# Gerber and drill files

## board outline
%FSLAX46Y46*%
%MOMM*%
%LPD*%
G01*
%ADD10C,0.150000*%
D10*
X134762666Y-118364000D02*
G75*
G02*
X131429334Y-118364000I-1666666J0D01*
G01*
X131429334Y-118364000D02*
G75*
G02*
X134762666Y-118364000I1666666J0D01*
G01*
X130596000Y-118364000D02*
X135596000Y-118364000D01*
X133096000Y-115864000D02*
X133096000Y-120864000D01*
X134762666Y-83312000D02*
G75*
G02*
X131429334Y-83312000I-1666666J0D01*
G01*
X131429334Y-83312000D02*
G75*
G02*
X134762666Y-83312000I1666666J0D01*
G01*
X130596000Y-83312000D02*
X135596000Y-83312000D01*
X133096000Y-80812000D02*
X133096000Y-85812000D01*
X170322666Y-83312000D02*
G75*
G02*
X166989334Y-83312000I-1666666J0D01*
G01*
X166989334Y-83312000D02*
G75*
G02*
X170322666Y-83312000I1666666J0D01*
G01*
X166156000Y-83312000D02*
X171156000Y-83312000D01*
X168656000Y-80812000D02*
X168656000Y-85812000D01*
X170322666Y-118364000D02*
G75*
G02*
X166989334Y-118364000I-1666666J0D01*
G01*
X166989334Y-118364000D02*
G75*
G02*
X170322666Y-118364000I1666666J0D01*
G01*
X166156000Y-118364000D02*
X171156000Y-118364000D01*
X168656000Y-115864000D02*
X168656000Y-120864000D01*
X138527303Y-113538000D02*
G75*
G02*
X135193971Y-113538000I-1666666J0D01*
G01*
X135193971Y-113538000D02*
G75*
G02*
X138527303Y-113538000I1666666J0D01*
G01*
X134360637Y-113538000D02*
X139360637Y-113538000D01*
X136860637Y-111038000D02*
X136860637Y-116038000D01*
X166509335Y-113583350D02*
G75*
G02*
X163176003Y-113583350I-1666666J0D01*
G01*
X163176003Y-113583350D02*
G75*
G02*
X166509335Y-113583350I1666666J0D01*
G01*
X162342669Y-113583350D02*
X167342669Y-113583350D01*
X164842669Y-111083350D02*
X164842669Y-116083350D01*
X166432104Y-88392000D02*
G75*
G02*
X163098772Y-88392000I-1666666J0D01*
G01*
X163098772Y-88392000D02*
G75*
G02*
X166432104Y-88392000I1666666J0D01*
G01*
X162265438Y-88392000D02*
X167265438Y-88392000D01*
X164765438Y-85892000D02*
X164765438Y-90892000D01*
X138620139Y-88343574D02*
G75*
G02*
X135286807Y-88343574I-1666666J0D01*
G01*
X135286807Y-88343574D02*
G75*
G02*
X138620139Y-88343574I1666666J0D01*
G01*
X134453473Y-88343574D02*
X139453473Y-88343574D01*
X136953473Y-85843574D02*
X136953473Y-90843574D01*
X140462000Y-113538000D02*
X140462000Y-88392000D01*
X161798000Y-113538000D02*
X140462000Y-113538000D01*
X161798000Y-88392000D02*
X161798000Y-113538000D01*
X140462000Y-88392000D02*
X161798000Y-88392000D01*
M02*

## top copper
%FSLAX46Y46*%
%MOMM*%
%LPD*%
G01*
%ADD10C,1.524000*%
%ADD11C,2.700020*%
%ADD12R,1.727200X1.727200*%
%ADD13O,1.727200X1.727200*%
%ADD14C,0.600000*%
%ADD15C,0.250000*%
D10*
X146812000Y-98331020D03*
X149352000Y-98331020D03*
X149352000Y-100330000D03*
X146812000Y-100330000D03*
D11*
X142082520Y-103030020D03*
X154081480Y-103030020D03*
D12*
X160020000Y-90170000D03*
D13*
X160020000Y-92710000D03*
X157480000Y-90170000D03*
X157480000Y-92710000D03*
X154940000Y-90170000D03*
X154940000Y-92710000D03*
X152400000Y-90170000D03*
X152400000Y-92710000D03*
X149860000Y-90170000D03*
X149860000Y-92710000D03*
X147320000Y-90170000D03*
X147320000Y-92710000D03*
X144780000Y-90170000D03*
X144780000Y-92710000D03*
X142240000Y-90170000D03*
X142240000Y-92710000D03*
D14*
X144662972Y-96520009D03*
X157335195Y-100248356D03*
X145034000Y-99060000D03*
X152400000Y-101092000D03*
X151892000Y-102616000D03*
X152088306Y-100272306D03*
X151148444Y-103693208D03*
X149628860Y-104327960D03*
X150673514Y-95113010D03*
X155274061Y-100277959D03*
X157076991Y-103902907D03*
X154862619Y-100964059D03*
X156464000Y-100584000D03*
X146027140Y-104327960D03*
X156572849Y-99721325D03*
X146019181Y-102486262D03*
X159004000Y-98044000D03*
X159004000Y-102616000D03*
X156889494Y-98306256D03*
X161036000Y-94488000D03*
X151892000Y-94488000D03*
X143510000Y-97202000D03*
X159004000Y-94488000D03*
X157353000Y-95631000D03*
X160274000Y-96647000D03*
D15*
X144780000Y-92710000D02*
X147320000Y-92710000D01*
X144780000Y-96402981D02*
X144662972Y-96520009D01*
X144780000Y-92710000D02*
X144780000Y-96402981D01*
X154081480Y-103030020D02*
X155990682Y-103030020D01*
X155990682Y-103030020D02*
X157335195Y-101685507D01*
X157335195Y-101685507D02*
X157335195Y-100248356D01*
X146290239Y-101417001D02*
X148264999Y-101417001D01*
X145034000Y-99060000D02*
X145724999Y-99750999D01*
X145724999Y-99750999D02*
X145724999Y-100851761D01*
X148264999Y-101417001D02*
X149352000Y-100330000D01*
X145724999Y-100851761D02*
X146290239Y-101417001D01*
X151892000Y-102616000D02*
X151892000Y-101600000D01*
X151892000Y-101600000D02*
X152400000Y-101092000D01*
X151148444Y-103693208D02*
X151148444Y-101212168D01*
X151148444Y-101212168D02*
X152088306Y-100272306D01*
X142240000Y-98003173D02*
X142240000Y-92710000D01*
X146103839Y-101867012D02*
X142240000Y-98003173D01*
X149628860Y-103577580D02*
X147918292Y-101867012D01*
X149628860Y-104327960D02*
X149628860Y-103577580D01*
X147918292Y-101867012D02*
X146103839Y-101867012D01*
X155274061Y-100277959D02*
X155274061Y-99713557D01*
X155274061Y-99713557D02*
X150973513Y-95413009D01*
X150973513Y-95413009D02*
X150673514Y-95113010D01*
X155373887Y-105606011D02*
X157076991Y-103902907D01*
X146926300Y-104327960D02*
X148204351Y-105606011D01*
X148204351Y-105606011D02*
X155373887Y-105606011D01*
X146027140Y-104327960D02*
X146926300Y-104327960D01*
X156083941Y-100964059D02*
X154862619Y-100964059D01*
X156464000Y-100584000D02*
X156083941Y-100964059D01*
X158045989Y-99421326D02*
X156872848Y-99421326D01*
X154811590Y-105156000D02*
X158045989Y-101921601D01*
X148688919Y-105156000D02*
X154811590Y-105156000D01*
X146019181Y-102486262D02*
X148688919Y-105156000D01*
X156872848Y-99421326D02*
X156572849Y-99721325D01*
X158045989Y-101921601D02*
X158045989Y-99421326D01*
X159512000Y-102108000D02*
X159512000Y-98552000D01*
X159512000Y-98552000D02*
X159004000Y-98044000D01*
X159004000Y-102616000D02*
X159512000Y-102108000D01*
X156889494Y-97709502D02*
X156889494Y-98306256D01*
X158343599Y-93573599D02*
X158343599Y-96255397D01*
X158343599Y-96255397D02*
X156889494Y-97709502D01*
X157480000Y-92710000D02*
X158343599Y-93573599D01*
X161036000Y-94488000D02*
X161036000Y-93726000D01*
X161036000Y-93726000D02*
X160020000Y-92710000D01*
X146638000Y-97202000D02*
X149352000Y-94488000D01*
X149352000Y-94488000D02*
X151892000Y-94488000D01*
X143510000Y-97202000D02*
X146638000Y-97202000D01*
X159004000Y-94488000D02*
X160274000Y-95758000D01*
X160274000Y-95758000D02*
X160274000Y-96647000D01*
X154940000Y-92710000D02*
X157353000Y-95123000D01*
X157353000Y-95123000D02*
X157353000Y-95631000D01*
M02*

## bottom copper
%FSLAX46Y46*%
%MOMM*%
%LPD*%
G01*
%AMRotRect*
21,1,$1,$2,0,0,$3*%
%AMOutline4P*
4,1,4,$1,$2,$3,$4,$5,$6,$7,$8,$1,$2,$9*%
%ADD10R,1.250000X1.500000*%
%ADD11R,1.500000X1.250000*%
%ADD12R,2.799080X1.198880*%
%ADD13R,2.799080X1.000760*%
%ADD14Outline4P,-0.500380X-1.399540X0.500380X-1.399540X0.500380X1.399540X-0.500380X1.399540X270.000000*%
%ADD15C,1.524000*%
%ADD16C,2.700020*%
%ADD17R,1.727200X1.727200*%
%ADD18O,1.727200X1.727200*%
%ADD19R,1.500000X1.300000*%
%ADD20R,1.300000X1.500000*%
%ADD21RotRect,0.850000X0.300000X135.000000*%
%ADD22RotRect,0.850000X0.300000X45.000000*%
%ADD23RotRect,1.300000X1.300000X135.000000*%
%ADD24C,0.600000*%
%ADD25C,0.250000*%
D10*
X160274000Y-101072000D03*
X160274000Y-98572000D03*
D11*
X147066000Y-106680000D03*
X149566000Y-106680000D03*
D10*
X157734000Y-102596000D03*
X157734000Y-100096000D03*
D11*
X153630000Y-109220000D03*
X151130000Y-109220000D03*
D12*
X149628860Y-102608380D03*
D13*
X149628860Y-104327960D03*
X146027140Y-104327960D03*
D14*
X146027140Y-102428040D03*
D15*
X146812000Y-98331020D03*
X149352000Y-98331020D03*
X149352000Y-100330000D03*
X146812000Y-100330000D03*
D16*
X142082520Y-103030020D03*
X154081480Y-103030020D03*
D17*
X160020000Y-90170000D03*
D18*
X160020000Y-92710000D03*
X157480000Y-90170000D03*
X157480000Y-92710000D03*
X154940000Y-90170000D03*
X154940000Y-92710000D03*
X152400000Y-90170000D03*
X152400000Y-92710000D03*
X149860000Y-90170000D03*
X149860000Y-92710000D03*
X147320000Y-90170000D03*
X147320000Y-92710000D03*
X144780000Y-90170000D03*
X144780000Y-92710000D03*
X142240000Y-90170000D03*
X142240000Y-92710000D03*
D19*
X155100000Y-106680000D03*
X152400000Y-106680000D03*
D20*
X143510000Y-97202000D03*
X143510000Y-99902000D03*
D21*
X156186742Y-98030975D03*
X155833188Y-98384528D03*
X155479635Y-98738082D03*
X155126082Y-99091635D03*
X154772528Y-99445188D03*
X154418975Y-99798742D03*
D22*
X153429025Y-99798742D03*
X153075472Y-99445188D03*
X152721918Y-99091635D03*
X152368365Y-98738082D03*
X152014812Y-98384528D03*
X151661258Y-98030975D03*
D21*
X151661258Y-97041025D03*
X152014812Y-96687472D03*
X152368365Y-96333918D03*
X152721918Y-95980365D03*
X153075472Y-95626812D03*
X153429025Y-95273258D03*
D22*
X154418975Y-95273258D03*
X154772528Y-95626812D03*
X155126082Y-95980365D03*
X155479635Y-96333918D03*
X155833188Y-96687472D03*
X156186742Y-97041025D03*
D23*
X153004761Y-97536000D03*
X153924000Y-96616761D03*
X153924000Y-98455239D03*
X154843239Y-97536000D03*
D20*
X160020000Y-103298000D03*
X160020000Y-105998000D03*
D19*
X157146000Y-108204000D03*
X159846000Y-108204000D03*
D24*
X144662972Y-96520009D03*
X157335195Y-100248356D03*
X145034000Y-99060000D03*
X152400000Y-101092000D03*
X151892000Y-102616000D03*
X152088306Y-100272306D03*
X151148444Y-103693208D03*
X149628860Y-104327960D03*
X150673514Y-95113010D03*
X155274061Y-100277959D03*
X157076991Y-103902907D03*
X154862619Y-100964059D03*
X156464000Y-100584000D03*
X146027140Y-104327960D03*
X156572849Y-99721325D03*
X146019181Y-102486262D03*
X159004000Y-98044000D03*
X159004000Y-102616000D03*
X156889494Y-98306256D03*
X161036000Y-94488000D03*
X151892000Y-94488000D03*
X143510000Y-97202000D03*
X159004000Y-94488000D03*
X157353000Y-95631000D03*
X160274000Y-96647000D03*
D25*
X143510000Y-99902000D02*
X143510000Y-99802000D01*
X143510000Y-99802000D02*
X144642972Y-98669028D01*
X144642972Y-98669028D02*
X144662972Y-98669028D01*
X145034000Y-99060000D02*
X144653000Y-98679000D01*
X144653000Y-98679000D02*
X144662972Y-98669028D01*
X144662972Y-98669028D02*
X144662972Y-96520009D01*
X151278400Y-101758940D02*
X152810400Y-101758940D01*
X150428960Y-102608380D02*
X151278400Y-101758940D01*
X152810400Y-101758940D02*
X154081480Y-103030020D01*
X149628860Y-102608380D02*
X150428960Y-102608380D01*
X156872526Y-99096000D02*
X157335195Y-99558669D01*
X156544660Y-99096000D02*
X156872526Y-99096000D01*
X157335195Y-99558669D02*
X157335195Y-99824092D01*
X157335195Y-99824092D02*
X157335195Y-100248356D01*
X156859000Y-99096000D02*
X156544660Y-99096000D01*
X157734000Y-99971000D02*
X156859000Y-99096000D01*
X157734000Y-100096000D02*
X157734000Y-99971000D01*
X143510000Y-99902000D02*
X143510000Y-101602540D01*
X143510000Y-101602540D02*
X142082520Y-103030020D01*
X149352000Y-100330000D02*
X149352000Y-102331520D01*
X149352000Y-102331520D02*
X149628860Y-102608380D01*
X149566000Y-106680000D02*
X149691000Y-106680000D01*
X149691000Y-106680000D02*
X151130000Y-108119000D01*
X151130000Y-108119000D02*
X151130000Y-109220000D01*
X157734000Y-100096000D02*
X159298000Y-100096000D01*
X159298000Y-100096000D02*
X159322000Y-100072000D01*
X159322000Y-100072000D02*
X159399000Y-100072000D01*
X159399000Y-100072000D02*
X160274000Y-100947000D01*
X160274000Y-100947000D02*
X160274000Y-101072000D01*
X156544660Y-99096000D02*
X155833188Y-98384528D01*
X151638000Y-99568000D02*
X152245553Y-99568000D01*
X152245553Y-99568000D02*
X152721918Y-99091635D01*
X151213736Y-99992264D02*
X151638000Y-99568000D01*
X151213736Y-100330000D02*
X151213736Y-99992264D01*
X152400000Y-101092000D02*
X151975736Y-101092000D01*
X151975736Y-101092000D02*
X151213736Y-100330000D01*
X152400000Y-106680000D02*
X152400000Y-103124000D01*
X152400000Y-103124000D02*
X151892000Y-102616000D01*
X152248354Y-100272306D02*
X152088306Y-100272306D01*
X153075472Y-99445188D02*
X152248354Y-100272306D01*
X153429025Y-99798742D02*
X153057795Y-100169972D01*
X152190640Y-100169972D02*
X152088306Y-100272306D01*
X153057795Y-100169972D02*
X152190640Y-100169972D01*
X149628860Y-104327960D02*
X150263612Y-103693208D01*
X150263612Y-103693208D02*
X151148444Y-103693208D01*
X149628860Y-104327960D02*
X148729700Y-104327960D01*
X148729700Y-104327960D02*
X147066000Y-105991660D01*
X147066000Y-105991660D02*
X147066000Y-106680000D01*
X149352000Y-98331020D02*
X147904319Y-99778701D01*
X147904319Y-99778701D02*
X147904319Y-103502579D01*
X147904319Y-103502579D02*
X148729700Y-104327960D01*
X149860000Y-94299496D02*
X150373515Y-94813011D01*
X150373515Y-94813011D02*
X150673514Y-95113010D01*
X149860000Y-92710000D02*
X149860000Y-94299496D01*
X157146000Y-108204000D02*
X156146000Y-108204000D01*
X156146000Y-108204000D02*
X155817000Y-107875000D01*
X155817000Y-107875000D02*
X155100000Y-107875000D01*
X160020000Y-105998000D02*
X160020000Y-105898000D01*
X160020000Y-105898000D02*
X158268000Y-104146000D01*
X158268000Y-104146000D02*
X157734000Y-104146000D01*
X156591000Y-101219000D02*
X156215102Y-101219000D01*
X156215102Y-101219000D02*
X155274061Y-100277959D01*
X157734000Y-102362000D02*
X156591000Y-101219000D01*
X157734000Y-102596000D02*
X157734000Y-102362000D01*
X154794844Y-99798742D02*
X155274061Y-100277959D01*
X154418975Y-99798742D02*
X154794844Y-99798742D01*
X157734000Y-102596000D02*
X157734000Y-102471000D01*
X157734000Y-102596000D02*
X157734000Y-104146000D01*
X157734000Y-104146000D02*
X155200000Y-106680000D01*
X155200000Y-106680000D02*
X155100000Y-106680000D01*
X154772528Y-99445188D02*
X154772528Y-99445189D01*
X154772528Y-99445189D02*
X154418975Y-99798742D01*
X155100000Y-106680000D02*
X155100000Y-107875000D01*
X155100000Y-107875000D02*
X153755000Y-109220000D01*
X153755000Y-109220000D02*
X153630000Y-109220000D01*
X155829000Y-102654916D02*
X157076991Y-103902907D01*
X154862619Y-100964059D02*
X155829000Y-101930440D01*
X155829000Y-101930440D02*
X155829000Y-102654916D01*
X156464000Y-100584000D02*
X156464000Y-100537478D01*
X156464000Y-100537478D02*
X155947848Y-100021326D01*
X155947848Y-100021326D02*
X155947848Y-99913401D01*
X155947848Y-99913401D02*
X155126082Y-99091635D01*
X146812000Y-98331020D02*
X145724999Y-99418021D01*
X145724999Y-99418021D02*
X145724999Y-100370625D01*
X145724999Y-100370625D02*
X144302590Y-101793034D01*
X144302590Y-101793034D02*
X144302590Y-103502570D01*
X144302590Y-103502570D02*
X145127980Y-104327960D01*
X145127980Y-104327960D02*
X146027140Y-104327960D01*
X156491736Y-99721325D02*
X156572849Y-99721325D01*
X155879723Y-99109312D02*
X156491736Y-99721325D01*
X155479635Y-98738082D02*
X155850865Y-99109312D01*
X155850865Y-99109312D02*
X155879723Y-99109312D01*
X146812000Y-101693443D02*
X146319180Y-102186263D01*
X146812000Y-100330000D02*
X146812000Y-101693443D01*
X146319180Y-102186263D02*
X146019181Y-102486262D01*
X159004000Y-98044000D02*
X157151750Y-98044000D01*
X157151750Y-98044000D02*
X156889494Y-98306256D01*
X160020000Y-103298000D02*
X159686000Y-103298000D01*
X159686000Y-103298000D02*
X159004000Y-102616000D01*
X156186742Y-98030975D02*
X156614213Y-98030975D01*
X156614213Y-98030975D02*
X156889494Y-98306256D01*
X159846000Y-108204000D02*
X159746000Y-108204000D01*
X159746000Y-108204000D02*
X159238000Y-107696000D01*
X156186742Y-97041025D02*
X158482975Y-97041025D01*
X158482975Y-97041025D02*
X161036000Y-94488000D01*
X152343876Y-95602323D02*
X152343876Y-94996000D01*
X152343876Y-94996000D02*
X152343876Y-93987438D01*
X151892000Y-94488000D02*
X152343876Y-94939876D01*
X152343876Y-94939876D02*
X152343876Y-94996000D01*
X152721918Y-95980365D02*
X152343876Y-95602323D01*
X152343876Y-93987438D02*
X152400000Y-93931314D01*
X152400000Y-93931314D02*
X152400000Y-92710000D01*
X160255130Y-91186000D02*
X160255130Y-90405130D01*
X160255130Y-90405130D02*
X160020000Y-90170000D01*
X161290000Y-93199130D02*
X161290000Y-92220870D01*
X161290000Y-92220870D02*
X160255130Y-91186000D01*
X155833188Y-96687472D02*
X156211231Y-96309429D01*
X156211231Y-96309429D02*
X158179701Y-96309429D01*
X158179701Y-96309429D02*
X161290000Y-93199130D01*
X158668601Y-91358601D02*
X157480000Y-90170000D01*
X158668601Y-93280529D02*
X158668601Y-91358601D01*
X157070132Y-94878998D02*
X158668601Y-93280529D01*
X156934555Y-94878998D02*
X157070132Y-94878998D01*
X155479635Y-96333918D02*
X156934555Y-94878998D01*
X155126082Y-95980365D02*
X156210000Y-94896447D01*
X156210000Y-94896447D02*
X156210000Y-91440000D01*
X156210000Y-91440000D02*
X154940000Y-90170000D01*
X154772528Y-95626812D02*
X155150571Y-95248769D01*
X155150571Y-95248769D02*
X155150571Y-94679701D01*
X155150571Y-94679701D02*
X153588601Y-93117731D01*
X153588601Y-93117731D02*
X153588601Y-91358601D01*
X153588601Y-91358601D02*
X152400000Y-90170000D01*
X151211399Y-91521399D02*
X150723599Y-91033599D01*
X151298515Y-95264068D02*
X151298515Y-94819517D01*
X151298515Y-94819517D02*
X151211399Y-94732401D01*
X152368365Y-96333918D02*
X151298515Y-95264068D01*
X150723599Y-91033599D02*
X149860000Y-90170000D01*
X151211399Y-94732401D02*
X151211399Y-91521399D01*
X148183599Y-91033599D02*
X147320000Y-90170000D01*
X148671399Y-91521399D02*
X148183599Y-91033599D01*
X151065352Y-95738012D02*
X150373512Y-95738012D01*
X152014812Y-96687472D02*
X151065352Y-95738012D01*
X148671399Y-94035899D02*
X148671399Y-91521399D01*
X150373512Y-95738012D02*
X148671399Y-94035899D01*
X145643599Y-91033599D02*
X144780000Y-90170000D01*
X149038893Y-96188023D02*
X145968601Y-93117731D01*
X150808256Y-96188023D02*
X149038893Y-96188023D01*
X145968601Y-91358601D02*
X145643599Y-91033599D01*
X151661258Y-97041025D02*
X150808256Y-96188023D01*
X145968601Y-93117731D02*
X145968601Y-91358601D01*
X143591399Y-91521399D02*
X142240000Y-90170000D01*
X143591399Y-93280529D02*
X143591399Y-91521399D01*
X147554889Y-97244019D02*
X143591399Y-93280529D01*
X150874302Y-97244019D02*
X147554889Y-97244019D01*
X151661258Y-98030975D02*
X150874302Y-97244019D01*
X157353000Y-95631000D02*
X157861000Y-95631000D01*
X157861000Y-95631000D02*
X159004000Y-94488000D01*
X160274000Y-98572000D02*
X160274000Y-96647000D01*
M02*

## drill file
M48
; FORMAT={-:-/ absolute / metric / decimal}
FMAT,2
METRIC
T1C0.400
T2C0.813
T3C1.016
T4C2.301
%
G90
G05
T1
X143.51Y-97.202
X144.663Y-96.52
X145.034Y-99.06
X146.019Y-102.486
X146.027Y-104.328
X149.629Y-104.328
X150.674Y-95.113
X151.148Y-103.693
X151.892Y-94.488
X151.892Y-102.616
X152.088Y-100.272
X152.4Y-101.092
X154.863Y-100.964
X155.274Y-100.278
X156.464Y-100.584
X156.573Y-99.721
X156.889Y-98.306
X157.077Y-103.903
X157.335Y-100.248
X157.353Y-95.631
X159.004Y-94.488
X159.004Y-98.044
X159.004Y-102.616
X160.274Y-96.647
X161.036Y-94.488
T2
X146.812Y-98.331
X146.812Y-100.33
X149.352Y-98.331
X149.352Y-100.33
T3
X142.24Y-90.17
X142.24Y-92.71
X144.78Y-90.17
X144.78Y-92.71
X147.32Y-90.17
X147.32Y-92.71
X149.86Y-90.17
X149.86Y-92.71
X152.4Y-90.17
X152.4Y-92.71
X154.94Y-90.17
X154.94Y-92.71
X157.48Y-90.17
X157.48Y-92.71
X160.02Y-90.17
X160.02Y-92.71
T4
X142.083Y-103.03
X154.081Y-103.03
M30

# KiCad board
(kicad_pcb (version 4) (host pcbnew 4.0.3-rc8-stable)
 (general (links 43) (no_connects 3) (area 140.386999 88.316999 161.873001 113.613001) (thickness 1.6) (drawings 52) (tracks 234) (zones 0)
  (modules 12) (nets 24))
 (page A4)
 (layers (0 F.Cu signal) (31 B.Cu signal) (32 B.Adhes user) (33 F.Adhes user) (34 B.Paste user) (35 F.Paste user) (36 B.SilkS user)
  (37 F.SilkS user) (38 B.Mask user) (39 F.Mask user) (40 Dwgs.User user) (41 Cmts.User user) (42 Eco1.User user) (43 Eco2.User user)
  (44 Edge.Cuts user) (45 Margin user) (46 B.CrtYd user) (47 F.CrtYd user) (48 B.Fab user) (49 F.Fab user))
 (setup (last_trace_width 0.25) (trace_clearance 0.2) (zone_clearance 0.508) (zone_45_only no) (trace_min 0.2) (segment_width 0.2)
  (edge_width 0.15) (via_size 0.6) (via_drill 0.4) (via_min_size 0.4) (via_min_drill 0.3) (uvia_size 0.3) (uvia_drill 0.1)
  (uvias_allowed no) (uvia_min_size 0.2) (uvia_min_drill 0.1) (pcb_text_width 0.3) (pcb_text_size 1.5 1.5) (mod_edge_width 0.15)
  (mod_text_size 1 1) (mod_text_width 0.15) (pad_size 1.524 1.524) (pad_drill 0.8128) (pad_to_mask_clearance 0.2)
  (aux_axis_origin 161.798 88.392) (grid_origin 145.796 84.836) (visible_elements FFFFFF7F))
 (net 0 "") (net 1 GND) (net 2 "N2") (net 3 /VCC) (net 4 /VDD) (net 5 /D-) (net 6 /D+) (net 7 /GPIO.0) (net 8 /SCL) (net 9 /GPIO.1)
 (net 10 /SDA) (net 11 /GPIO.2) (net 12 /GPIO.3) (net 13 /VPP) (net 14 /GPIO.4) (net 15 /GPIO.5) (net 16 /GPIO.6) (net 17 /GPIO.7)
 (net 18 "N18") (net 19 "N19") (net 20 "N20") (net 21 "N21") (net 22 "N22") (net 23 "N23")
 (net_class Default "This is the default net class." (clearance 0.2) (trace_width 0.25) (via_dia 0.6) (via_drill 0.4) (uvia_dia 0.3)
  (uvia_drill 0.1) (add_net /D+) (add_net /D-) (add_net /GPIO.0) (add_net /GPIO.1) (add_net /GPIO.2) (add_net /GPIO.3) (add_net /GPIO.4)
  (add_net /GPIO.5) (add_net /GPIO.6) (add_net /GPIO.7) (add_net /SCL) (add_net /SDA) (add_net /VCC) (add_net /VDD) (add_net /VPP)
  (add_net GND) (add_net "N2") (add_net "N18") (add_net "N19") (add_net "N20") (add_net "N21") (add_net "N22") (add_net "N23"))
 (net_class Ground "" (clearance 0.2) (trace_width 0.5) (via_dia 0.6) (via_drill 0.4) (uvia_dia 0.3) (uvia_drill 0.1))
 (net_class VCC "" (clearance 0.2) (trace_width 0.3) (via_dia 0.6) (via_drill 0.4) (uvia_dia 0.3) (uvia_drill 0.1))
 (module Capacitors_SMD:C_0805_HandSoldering (layer B.Cu) (at 160.274 99.822 90)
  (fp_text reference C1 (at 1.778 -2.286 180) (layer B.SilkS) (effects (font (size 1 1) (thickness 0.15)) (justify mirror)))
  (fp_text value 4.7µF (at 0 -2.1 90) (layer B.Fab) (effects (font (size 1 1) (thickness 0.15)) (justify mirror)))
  (pad 1 smd rect (at -1.25 0 90) (size 1.5 1.25) (layers B.Cu B.Paste B.Mask) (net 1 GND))
  (pad 2 smd rect (at 1.25 0 90) (size 1.5 1.25) (layers B.Cu B.Paste B.Mask) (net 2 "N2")))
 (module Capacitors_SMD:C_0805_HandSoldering (layer B.Cu) (at 148.316 106.68)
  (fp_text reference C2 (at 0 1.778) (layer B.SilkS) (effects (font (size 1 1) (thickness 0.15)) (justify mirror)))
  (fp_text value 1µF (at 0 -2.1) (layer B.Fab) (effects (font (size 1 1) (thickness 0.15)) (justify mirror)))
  (pad 1 smd rect (at -1.25 0) (size 1.5 1.25) (layers B.Cu B.Paste B.Mask) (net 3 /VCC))
  (pad 2 smd rect (at 1.25 0) (size 1.5 1.25) (layers B.Cu B.Paste B.Mask) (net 1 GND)))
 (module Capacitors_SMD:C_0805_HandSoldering (layer B.Cu) (at 157.734 101.346 90)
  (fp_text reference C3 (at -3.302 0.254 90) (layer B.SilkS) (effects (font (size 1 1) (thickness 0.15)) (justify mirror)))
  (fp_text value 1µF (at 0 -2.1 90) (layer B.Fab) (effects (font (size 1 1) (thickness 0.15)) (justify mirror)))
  (pad 1 smd rect (at -1.25 0 90) (size 1.5 1.25) (layers B.Cu B.Paste B.Mask) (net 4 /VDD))
  (pad 2 smd rect (at 1.25 0 90) (size 1.5 1.25) (layers B.Cu B.Paste B.Mask) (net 1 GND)))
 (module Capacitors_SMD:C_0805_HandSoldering (layer B.Cu) (at 152.38 109.22 180)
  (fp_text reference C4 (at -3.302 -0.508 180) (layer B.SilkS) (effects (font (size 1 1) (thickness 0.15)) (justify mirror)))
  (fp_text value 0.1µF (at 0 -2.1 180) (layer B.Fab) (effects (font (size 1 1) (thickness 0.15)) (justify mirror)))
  (pad 1 smd rect (at -1.25 0 180) (size 1.5 1.25) (layers B.Cu B.Paste B.Mask) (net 4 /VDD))
  (pad 2 smd rect (at 1.25 0 180) (size 1.5 1.25) (layers B.Cu B.Paste B.Mask) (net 1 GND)))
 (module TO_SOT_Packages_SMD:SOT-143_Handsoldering (layer B.Cu) (at 147.828 103.378 270)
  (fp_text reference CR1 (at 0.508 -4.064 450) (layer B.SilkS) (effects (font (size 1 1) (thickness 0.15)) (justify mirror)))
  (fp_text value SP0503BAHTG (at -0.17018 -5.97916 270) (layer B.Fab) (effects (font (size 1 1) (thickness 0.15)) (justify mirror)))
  (pad 1 smd rect (at -0.76962 -1.80086 270) (size 1.19888 2.79908) (layers B.Cu B.Paste B.Mask) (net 1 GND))
  (pad 2 smd rect (at 0.94996 -1.80086 270) (size 1.00076 2.79908) (layers B.Cu B.Paste B.Mask) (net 3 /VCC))
  (pad 3 smd rect (at 0.94996 1.80086 270) (size 1.00076 2.79908) (layers B.Cu B.Paste B.Mask) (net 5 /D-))
  (pad 4 smd trapezoid (at -0.94996 1.80086 270) (size 1.00076 2.79908) (layers B.Cu B.Paste B.Mask) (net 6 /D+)))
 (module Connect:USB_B (layer F.Cu) (at 149.352 98.33102 270)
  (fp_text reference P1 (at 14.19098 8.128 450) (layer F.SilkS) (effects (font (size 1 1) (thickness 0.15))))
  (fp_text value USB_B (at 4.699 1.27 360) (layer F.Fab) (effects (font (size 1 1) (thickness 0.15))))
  (pad 2 thru_hole circle (at 0 2.54 180) (size 1.524 1.524) (drill 0.8128) (layers *.Cu *.Mask F.SilkS) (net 5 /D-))
  (pad 1 thru_hole circle (at 0 0 180) (size 1.524 1.524) (drill 0.8128) (layers *.Cu *.Mask F.SilkS) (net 3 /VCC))
  (pad 4 thru_hole circle (at 1.99898 0 180) (size 1.524 1.524) (drill 0.8128) (layers *.Cu *.Mask F.SilkS) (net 1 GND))
  (pad 3 thru_hole circle (at 1.99898 2.54 180) (size 1.524 1.524) (drill 0.8128) (layers *.Cu *.Mask F.SilkS) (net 6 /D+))
  (pad 5 thru_hole circle (at 4.699 7.26948 180) (size 2.70002 2.70002) (drill 2.30124) (layers *.Cu *.Mask F.SilkS) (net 1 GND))
  (pad 5 thru_hole circle (at 4.699 -4.72948 180) (size 2.70002 2.70002) (drill 2.30124) (layers *.Cu *.Mask F.SilkS) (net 1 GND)))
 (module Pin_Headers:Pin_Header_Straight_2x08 (layer F.Cu) (at 160.02 90.17 270)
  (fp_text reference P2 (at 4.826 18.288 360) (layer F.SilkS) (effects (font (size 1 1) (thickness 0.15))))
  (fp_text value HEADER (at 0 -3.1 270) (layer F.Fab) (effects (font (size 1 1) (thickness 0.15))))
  (pad 1 thru_hole rect (at 0 0 270) (size 1.7272 1.7272) (drill 1.016) (layers *.Cu *.Mask F.SilkS) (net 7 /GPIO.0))
  (pad 2 thru_hole oval (at 2.54 0 270) (size 1.7272 1.7272) (drill 1.016) (layers *.Cu *.Mask F.SilkS) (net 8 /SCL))
  (pad 3 thru_hole oval (at 0 2.54 270) (size 1.7272 1.7272) (drill 1.016) (layers *.Cu *.Mask F.SilkS) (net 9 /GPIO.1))
  (pad 4 thru_hole oval (at 2.54 2.54 270) (size 1.7272 1.7272) (drill 1.016) (layers *.Cu *.Mask F.SilkS) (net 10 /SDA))
  (pad 5 thru_hole oval (at 0 5.08 270) (size 1.7272 1.7272) (drill 1.016) (layers *.Cu *.Mask F.SilkS) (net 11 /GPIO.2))
  (pad 6 thru_hole oval (at 2.54 5.08 270) (size 1.7272 1.7272) (drill 1.016) (layers *.Cu *.Mask F.SilkS) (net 2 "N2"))
  (pad 7 thru_hole oval (at 0 7.62 270) (size 1.7272 1.7272) (drill 1.016) (layers *.Cu *.Mask F.SilkS) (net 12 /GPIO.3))
  (pad 8 thru_hole oval (at 2.54 7.62 270) (size 1.7272 1.7272) (drill 1.016) (layers *.Cu *.Mask F.SilkS) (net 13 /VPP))
  (pad 9 thru_hole oval (at 0 10.16 270) (size 1.7272 1.7272) (drill 1.016) (layers *.Cu *.Mask F.SilkS) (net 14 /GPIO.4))
  (pad 10 thru_hole oval (at 2.54 10.16 270) (size 1.7272 1.7272) (drill 1.016) (layers *.Cu *.Mask F.SilkS) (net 4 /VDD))
  (pad 11 thru_hole oval (at 0 12.7 270) (size 1.7272 1.7272) (drill 1.016) (layers *.Cu *.Mask F.SilkS) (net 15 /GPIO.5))
  (pad 12 thru_hole oval (at 2.54 12.7 270) (size 1.7272 1.7272) (drill 1.016) (layers *.Cu *.Mask F.SilkS) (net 1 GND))
  (pad 13 thru_hole oval (at 0 15.24 270) (size 1.7272 1.7272) (drill 1.016) (layers *.Cu *.Mask F.SilkS) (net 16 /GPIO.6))
  (pad 14 thru_hole oval (at 2.54 15.24 270) (size 1.7272 1.7272) (drill 1.016) (layers *.Cu *.Mask F.SilkS) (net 1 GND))
  (pad 15 thru_hole oval (at 0 17.78 270) (size 1.7272 1.7272) (drill 1.016) (layers *.Cu *.Mask F.SilkS) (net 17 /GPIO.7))
  (pad 16 thru_hole oval (at 2.54 17.78 270) (size 1.7272 1.7272) (drill 1.016) (layers *.Cu *.Mask F.SilkS) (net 3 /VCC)))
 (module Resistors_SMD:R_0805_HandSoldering (layer B.Cu) (at 153.75 106.68 180)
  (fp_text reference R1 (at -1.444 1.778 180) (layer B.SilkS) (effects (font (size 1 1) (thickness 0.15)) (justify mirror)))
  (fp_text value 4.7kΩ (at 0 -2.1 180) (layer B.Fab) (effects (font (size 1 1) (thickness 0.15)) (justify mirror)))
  (pad 1 smd rect (at -1.35 0 180) (size 1.5 1.3) (layers B.Cu B.Paste B.Mask) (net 4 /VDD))
  (pad 2 smd rect (at 1.35 0 180) (size 1.5 1.3) (layers B.Cu B.Paste B.Mask) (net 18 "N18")))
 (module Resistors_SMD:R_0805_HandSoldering (layer B.Cu) (at 143.51 98.552 270)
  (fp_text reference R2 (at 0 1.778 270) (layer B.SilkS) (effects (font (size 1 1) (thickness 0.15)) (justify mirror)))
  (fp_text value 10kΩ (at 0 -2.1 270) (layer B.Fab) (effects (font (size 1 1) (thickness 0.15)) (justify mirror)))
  (pad 1 smd rect (at -1.35 0 270) (size 1.5 1.3) (layers B.Cu B.Paste B.Mask) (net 13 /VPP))
  (pad 2 smd rect (at 1.35 0 270) (size 1.5 1.3) (layers B.Cu B.Paste B.Mask) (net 1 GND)))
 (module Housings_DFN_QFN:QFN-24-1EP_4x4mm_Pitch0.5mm (layer B.Cu) (at 153.924 97.536 135)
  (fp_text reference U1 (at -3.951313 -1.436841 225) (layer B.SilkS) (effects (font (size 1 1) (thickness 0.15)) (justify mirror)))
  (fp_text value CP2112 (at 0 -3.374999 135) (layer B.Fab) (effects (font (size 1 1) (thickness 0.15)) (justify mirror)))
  (pad 1 smd rect (at -1.95 1.25 135) (size 0.85 0.3) (layers B.Cu B.Paste B.Mask) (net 10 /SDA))
  (pad 2 smd rect (at -1.95 0.75 135) (size 0.85 0.3) (layers B.Cu B.Paste B.Mask) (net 1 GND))
  (pad 3 smd rect (at -1.95 0.25 135) (size 0.85 0.3) (layers B.Cu B.Paste B.Mask) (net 6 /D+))
  (pad 4 smd rect (at -1.95 -0.25 135) (size 0.85 0.3) (layers B.Cu B.Paste B.Mask) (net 5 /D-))
  (pad 5 smd rect (at -1.95 -0.75 135) (size 0.85 0.3) (layers B.Cu B.Paste B.Mask) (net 4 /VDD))
  (pad 6 smd rect (at -1.95 -1.25 135) (size 0.85 0.3) (layers B.Cu B.Paste B.Mask) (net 4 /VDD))
  (pad 7 smd rect (at -1.25 -1.95 45) (size 0.85 0.3) (layers B.Cu B.Paste B.Mask) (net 3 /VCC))
  (pad 8 smd rect (at -0.75 -1.95 45) (size 0.85 0.3) (layers B.Cu B.Paste B.Mask) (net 3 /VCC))
  (pad 9 smd rect (at -0.25 -1.95 45) (size 0.85 0.3) (layers B.Cu B.Paste B.Mask) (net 18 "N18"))
  (pad 10 smd rect (at 0.25 -1.95 45) (size 0.85 0.3) (layers B.Cu B.Paste B.Mask) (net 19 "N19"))
  (pad 11 smd rect (at 0.75 -1.95 45) (size 0.85 0.3) (layers B.Cu B.Paste B.Mask) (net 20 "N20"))
  (pad 12 smd rect (at 1.25 -1.95 45) (size 0.85 0.3) (layers B.Cu B.Paste B.Mask) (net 17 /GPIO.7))
  (pad 13 smd rect (at 1.95 -1.25 135) (size 0.85 0.3) (layers B.Cu B.Paste B.Mask) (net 16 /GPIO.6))
  (pad 14 smd rect (at 1.95 -0.75 135) (size 0.85 0.3) (layers B.Cu B.Paste B.Mask) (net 15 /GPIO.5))
  (pad 15 smd rect (at 1.95 -0.25 135) (size 0.85 0.3) (layers B.Cu B.Paste B.Mask) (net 14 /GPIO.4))
  (pad 16 smd rect (at 1.95 0.25 135) (size 0.85 0.3) (layers B.Cu B.Paste B.Mask) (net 13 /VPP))
  (pad 17 smd rect (at 1.95 0.75 135) (size 0.85 0.3) (layers B.Cu B.Paste B.Mask) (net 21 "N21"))
  (pad 18 smd rect (at 1.95 1.25 135) (size 0.85 0.3) (layers B.Cu B.Paste B.Mask) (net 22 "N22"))
  (pad 19 smd rect (at 1.25 1.95 45) (size 0.85 0.3) (layers B.Cu B.Paste B.Mask) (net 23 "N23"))
  (pad 20 smd rect (at 0.75 1.95 45) (size 0.85 0.3) (layers B.Cu B.Paste B.Mask) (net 12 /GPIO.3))
  (pad 21 smd rect (at 0.25 1.95 45) (size 0.85 0.3) (layers B.Cu B.Paste B.Mask) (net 11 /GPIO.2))
  (pad 22 smd rect (at -0.25 1.95 45) (size 0.85 0.3) (layers B.Cu B.Paste B.Mask) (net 9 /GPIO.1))
  (pad 23 smd rect (at -0.75 1.95 45) (size 0.85 0.3) (layers B.Cu B.Paste B.Mask) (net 7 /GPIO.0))
  (pad 24 smd rect (at -1.25 1.95 45) (size 0.85 0.3) (layers B.Cu B.Paste B.Mask) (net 8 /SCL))
  (pad 25 smd rect (at 0.65 -0.65 135) (size 1.3 1.3) (layers B.Cu B.Paste B.Mask) (solder_paste_margin_ratio -0.2))
  (pad 25 smd rect (at 0.65 0.65 135) (size 1.3 1.3) (layers B.Cu B.Paste B.Mask) (solder_paste_margin_ratio -0.2))
  (pad 25 smd rect (at -0.65 -0.65 135) (size 1.3 1.3) (layers B.Cu B.Paste B.Mask) (solder_paste_margin_ratio -0.2))
  (pad 25 smd rect (at -0.65 0.65 135) (size 1.3 1.3) (layers B.Cu B.Paste B.Mask) (solder_paste_margin_ratio -0.2)))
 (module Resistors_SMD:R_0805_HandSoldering (layer B.Cu) (at 160.02 104.648 270)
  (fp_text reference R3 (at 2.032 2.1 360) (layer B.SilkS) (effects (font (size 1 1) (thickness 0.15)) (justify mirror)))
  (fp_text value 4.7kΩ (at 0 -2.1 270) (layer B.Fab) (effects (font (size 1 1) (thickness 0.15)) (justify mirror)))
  (pad 1 smd rect (at -1.35 0 270) (size 1.5 1.3) (layers B.Cu B.Paste B.Mask) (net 10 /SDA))
  (pad 2 smd rect (at 1.35 0 270) (size 1.5 1.3) (layers B.Cu B.Paste B.Mask) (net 4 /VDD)))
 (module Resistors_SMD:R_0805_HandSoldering (layer B.Cu) (at 158.496 108.204)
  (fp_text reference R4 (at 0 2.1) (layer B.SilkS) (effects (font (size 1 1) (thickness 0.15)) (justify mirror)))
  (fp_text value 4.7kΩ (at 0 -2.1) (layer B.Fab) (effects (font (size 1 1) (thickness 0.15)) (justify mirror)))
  (pad 1 smd rect (at -1.35 0) (size 1.5 1.3) (layers B.Cu B.Paste B.Mask) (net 4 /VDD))
  (pad 2 smd rect (at 1.35 0) (size 1.5 1.3) (layers B.Cu B.Paste B.Mask) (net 8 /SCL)))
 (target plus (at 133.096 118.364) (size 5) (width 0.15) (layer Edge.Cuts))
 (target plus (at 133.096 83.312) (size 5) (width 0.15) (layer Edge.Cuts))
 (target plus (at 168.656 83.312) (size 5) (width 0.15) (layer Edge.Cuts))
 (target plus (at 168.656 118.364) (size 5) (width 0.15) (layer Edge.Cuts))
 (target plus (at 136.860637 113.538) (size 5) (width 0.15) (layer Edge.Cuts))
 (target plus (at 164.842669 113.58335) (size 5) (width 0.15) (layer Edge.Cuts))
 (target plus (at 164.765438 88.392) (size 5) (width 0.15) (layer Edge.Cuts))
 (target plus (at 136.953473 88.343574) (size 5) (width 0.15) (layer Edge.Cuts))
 (gr_line (start 140.462 113.538) (end 140.462 88.392) (layer Edge.Cuts) (width 0.15))
 (gr_line (start 161.798 113.538) (end 140.462 113.538) (layer Edge.Cuts) (width 0.15))
 (gr_line (start 161.798 88.392) (end 161.798 113.538) (layer Edge.Cuts) (width 0.15))
 (gr_line (start 140.462 88.392) (end 161.798 88.392) (layer Edge.Cuts) (width 0.15))
 (segment (start 143.51 99.902) (end 143.51 99.802) (width 0.25) (layer B.Cu) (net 1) (status 30))
 (segment (start 143.51 99.802) (end 144.642972 98.669028) (width 0.25) (layer B.Cu) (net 1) (status 10))
 (segment (start 144.642972 98.669028) (end 144.662972 98.669028) (width 0.25) (layer B.Cu) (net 1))
 (segment (start 145.034 99.06) (end 144.653 98.679) (width 0.25) (layer B.Cu) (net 1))
 (segment (start 144.653 98.679) (end 144.662972 98.669028) (width 0.25) (layer B.Cu) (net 1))
 (segment (start 144.662972 98.669028) (end 144.662972 96.520009) (width 0.25) (layer B.Cu) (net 1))
 (segment (start 144.78 92.71) (end 147.32 92.71) (width 0.25) (layer F.Cu) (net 1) (status 30))
 (segment (start 144.78 96.402981) (end 144.662972 96.520009) (width 0.25) (layer F.Cu) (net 1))
 (segment (start 144.78 92.71) (end 144.78 96.402981) (width 0.25) (layer F.Cu) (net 1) (status 10))
 (via (at 144.662972 96.520009) (size 0.6) (drill 0.4) (layers F.Cu B.Cu) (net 1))
 (segment (start 151.2784 101.75894) (end 152.8104 101.75894) (width 0.25) (layer B.Cu) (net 1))
 (segment (start 150.42896 102.60838) (end 151.2784 101.75894) (width 0.25) (layer B.Cu) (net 1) (status 10))
 (segment (start 152.8104 101.75894) (end 154.08148 103.03002) (width 0.25) (layer B.Cu) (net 1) (status 20))
 (segment (start 149.62886 102.60838) (end 150.42896 102.60838) (width 0.25) (layer B.Cu) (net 1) (status 30))
 (segment (start 156.872526 99.096) (end 157.335195 99.558669) (width 0.25) (layer B.Cu) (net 1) (status 20))
 (segment (start 156.54466 99.096) (end 156.872526 99.096) (width 0.25) (layer B.Cu) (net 1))
 (segment (start 157.335195 99.558669) (end 157.335195 99.824092) (width 0.25) (layer B.Cu) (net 1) (status 30))
 (segment (start 157.335195 99.824092) (end 157.335195 100.248356) (width 0.25) (layer B.Cu) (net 1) (status 30))
 (segment (start 154.08148 103.03002) (end 155.990682 103.03002) (width 0.25) (layer F.Cu) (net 1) (status 10))
 (via (at 157.335195 100.248356) (size 0.6) (drill 0.4) (layers F.Cu B.Cu) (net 1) (status 30))
 (segment (start 155.990682 103.03002) (end 157.335195 101.685507) (width 0.25) (layer F.Cu) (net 1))
 (segment (start 157.335195 101.685507) (end 157.335195 100.248356) (width 0.25) (layer F.Cu) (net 1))
 (segment (start 156.859 99.096) (end 156.54466 99.096) (width 0.25) (layer B.Cu) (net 1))
 (segment (start 157.734 99.971) (end 156.859 99.096) (width 0.25) (layer B.Cu) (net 1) (status 10))
 (segment (start 157.734 100.096) (end 157.734 99.971) (width 0.25) (layer B.Cu) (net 1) (status 30))
 (segment (start 146.290239 101.417001) (end 148.264999 101.417001) (width 0.25) (layer F.Cu) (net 1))
 (segment (start 145.034 99.06) (end 145.724999 99.750999) (width 0.25) (layer F.Cu) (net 1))
 (segment (start 145.724999 99.750999) (end 145.724999 100.851761) (width 0.25) (layer F.Cu) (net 1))
 (segment (start 148.264999 101.417001) (end 149.352 100.33) (width 0.25) (layer F.Cu) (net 1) (status 20))
 (segment (start 145.724999 100.851761) (end 146.290239 101.417001) (width 0.25) (layer F.Cu) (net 1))
 (via (at 145.034 99.06) (size 0.6) (drill 0.4) (layers F.Cu B.Cu) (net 1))
 (segment (start 143.51 99.902) (end 143.51 101.60254) (width 0.25) (layer B.Cu) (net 1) (status 10))
 (segment (start 143.51 101.60254) (end 142.08252 103.03002) (width 0.25) (layer B.Cu) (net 1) (status 20))
 (segment (start 149.352 100.33) (end 149.352 102.33152) (width 0.25) (layer B.Cu) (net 1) (status 30))
 (segment (start 149.352 102.33152) (end 149.62886 102.60838) (width 0.25) (layer B.Cu) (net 1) (status 30))
 (segment (start 149.566 106.68) (end 149.691 106.68) (width 0.25) (layer B.Cu) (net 1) (status 30))
 (segment (start 149.691 106.68) (end 151.13 108.119) (width 0.25) (layer B.Cu) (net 1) (status 10))
 (segment (start 151.13 108.119) (end 151.13 109.22) (width 0.25) (layer B.Cu) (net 1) (status 20))
 (segment (start 157.734 100.096) (end 159.298 100.096) (width 0.25) (layer B.Cu) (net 1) (status 10))
 (segment (start 159.298 100.096) (end 159.322 100.072) (width 0.25) (layer B.Cu) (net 1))
 (segment (start 159.322 100.072) (end 159.399 100.072) (width 0.25) (layer B.Cu) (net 1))
 (segment (start 159.399 100.072) (end 160.274 100.947) (width 0.25) (layer B.Cu) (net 1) (status 20))
 (segment (start 160.274 100.947) (end 160.274 101.072) (width 0.25) (layer B.Cu) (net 1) (status 30))
 (segment (start 156.54466 99.096) (end 155.833188 98.384528) (width 0.25) (layer B.Cu) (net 1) (status 20))
 (segment (start 151.638 99.568) (end 152.245553 99.568) (width 0.25) (layer B.Cu) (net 18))
 (segment (start 152.245553 99.568) (end 152.721918 99.091635) (width 0.25) (layer B.Cu) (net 18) (status 20))
 (segment (start 151.213736 99.992264) (end 151.638 99.568) (width 0.25) (layer B.Cu) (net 18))
 (segment (start 151.213736 100.33) (end 151.213736 99.992264) (width 0.25) (layer B.Cu) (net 18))
 (segment (start 152.4 101.092) (end 151.975736 101.092) (width 0.25) (layer B.Cu) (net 18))
 (segment (start 151.975736 101.092) (end 151.213736 100.33) (width 0.25) (layer B.Cu) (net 18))
 (segment (start 151.892 102.616) (end 151.892 101.6) (width 0.25) (layer F.Cu) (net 18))
 (via (at 152.4 101.092) (size 0.6) (drill 0.4) (layers F.Cu B.Cu) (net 18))
 (segment (start 151.892 101.6) (end 152.4 101.092) (width 0.25) (layer F.Cu) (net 18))
 (via (at 151.892 102.616) (size 0.6) (drill 0.4) (layers F.Cu B.Cu) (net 18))
 (segment (start 152.4 106.68) (end 152.4 103.124) (width 0.25) (layer B.Cu) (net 18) (status 10))
 (segment (start 152.4 103.124) (end 151.892 102.616) (width 0.25) (layer B.Cu) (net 18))
 (segment (start 152.248354 100.272306) (end 152.088306 100.272306) (width 0.25) (layer B.Cu) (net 3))
 (via (at 152.088306 100.272306) (size 0.6) (drill 0.4) (layers F.Cu B.Cu) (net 3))
 (segment (start 153.075472 99.445188) (end 152.248354 100.272306) (width 0.25) (layer B.Cu) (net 3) (status 10))
 (segment (start 151.148444 103.693208) (end 151.148444 101.212168) (width 0.25) (layer F.Cu) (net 3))
 (segment (start 151.148444 101.212168) (end 152.088306 100.272306) (width 0.25) (layer F.Cu) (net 3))
 (segment (start 153.429025 99.798742) (end 153.057795 100.169972) (width 0.25) (layer B.Cu) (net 3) (status 10))
 (segment (start 152.19064 100.169972) (end 152.088306 100.272306) (width 0.25) (layer B.Cu) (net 3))
 (segment (start 153.057795 100.169972) (end 152.19064 100.169972) (width 0.25) (layer B.Cu) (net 3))
 (via (at 151.148444 103.693208) (size 0.6) (drill 0.4) (layers F.Cu B.Cu) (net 3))
 (segment (start 149.62886 104.32796) (end 150.263612 103.693208) (width 0.25) (layer B.Cu) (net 3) (status 10))
 (segment (start 150.263612 103.693208) (end 151.148444 103.693208) (width 0.25) (layer B.Cu) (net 3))
 (segment (start 142.24 98.003173) (end 142.24 92.71) (width 0.25) (layer F.Cu) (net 3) (status 20))
 (segment (start 146.103839 101.867012) (end 142.24 98.003173) (width 0.25) (layer F.Cu) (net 3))
 (segment (start 149.62886 103.57758) (end 147.918292 101.867012) (width 0.25) (layer F.Cu) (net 3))
 (segment (start 149.62886 104.32796) (end 149.62886 103.57758) (width 0.25) (layer F.Cu) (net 3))
 (segment (start 147.918292 101.867012) (end 146.103839 101.867012) (width 0.25) (layer F.Cu) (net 3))
 (via (at 149.62886 104.32796) (size 0.6) (drill 0.4) (layers F.Cu B.Cu) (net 3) (status 30))
 (segment (start 149.62886 104.32796) (end 148.7297 104.32796) (width 0.25) (layer B.Cu) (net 3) (status 30))
 (segment (start 148.7297 104.32796) (end 147.066 105.99166) (width 0.25) (layer B.Cu) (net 3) (status 10))
 (segment (start 147.066 105.99166) (end 147.066 106.68) (width 0.25) (layer B.Cu) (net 3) (status 20))
 (segment (start 149.352 98.33102) (end 147.904319 99.778701) (width 0.25) (layer B.Cu) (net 3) (status 10))
 (segment (start 147.904319 99.778701) (end 147.904319 103.502579) (width 0.25) (layer B.Cu) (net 3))
 (segment (start 147.904319 103.502579) (end 148.7297 104.32796) (width 0.25) (layer B.Cu) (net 3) (status 20))
 (segment (start 149.86 94.299496) (end 150.373515 94.813011) (width 0.25) (layer B.Cu) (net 4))
 (segment (start 150.373515 94.813011) (end 150.673514 95.11301) (width 0.25) (layer B.Cu) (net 4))
 (segment (start 155.274061 100.277959) (end 155.274061 99.713557) (width 0.25) (layer F.Cu) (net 4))
 (segment (start 149.86 92.71) (end 149.86 94.299496) (width 0.25) (layer B.Cu) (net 4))
 (via (at 150.673514 95.11301) (size 0.6) (drill 0.4) (layers F.Cu B.Cu) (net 4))
 (segment (start 155.274061 99.713557) (end 150.973513 95.413009) (width 0.25) (layer F.Cu) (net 4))
 (segment (start 150.973513 95.413009) (end 150.673514 95.11301) (width 0.25) (layer F.Cu) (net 4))
 (segment (start 157.146 108.204) (end 156.146 108.204) (width 0.25) (layer B.Cu) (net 4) (status 10))
 (segment (start 156.146 108.204) (end 155.817 107.875) (width 0.25) (layer B.Cu) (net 4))
 (segment (start 155.817 107.875) (end 155.1 107.875) (width 0.25) (layer B.Cu) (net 4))
 (segment (start 160.02 105.998) (end 160.02 105.898) (width 0.25) (layer B.Cu) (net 4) (status 30))
 (segment (start 160.02 105.898) (end 158.268 104.146) (width 0.25) (layer B.Cu) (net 4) (status 10))
 (segment (start 158.268 104.146) (end 157.734 104.146) (width 0.25) (layer B.Cu) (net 4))
 (segment (start 156.591 101.219) (end 156.215102 101.219) (width 0.25) (layer B.Cu) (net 4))
 (segment (start 156.215102 101.219) (end 155.274061 100.277959) (width 0.25) (layer B.Cu) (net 4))
 (segment (start 157.734 102.362) (end 156.591 101.219) (width 0.25) (layer B.Cu) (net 4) (status 10))
 (segment (start 157.734 102.596) (end 157.734 102.362) (width 0.25) (layer B.Cu) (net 4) (status 30))
 (segment (start 154.794844 99.798742) (end 155.274061 100.277959) (width 0.25) (layer B.Cu) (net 4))
 (segment (start 154.418975 99.798742) (end 154.794844 99.798742) (width 0.25) (layer B.Cu) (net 4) (status 10))
 (via (at 155.274061 100.277959) (size 0.6) (drill 0.4) (layers F.Cu B.Cu) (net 4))
 (segment (start 157.734 102.596) (end 157.734 102.471) (width 0.25) (layer B.Cu) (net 4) (status 30))
 (segment (start 157.734 102.596) (end 157.734 104.146) (width 0.25) (layer B.Cu) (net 4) (status 10))
 (segment (start 157.734 104.146) (end 155.2 106.68) (width 0.25) (layer B.Cu) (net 4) (status 20))
 (segment (start 155.2 106.68) (end 155.1 106.68) (width 0.25) (layer B.Cu) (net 4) (status 30))
 (segment (start 154.772528 99.445188) (end 154.772528 99.445189) (width 0.25) (layer B.Cu) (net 4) (status 30))
 (segment (start 154.772528 99.445189) (end 154.418975 99.798742) (width 0.25) (layer B.Cu) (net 4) (status 30))
 (segment (start 155.1 106.68) (end 155.1 107.875) (width 0.25) (layer B.Cu) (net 4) (status 10))
 (segment (start 155.1 107.875) (end 153.755 109.22) (width 0.25) (layer B.Cu) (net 4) (status 20))
 (segment (start 153.755 109.22) (end 153.63 109.22) (width 0.25) (layer B.Cu) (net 4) (status 30))
 (segment (start 155.373887 105.606011) (end 157.076991 103.902907) (width 0.25) (layer F.Cu) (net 5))
 (segment (start 146.9263 104.32796) (end 148.204351 105.606011) (width 0.25) (layer F.Cu) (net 5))
 (segment (start 148.204351 105.606011) (end 155.373887 105.606011) (width 0.25) (layer F.Cu) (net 5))
 (segment (start 146.02714 104.32796) (end 146.9263 104.32796) (width 0.25) (layer F.Cu) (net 5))
 (segment (start 155.829 102.654916) (end 157.076991 103.902907) (width 0.25) (layer B.Cu) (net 5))
 (segment (start 154.862619 100.964059) (end 155.829 101.93044) (width 0.25) (layer B.Cu) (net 5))
 (via (at 157.076991 103.902907) (size 0.6) (drill 0.4) (layers F.Cu B.Cu) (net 5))
 (segment (start 155.829 101.93044) (end 155.829 102.654916) (width 0.25) (layer B.Cu) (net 5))
 (segment (start 156.464 100.584) (end 156.464 100.537478) (width 0.25) (layer B.Cu) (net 5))
 (segment (start 156.464 100.537478) (end 155.947848 100.021326) (width 0.25) (layer B.Cu) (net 5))
 (segment (start 155.947848 100.021326) (end 155.947848 99.913401) (width 0.25) (layer B.Cu) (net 5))
 (segment (start 155.947848 99.913401) (end 155.126082 99.091635) (width 0.25) (layer B.Cu) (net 5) (status 20))
 (segment (start 156.083941 100.964059) (end 154.862619 100.964059) (width 0.25) (layer F.Cu) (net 5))
 (segment (start 156.464 100.584) (end 156.083941 100.964059) (width 0.25) (layer F.Cu) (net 5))
 (via (at 154.862619 100.964059) (size 0.6) (drill 0.4) (layers F.Cu B.Cu) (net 5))
 (via (at 156.464 100.584) (size 0.6) (drill 0.4) (layers F.Cu B.Cu) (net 5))
 (via (at 146.02714 104.32796) (size 0.6) (drill 0.4) (layers F.Cu B.Cu) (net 5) (status 30))
 (segment (start 146.812 98.33102) (end 145.724999 99.418021) (width 0.25) (layer B.Cu) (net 5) (status 10))
 (segment (start 145.724999 99.418021) (end 145.724999 100.370625) (width 0.25) (layer B.Cu) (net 5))
 (segment (start 145.724999 100.370625) (end 144.30259 101.793034) (width 0.25) (layer B.Cu) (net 5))
 (segment (start 144.30259 101.793034) (end 144.30259 103.50257) (width 0.25) (layer B.Cu) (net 5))
 (segment (start 144.30259 103.50257) (end 145.12798 104.32796) (width 0.25) (layer B.Cu) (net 5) (status 20))
 (segment (start 145.12798 104.32796) (end 146.02714 104.32796) (width 0.25) (layer B.Cu) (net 5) (status 30))
 (segment (start 158.045989 99.421326) (end 156.872848 99.421326) (width 0.25) (layer F.Cu) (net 6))
 (segment (start 154.81159 105.156) (end 158.045989 101.921601) (width 0.25) (layer F.Cu) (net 6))
 (segment (start 148.688919 105.156) (end 154.81159 105.156) (width 0.25) (layer F.Cu) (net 6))
 (segment (start 146.019181 102.486262) (end 148.688919 105.156) (width 0.25) (layer F.Cu) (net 6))
 (segment (start 156.872848 99.421326) (end 156.572849 99.721325) (width 0.25) (layer F.Cu) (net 6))
 (segment (start 158.045989 101.921601) (end 158.045989 99.421326) (width 0.25) (layer F.Cu) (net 6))
 (via (at 156.572849 99.721325) (size 0.6) (drill 0.4) (layers F.Cu B.Cu) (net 6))
 (segment (start 156.491736 99.721325) (end 156.572849 99.721325) (width 0.25) (layer B.Cu) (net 6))
 (segment (start 155.879723 99.109312) (end 156.491736 99.721325) (width 0.25) (layer B.Cu) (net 6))
 (segment (start 155.479635 98.738082) (end 155.850865 99.109312) (width 0.25) (layer B.Cu) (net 6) (status 10))
 (segment (start 155.850865 99.109312) (end 155.879723 99.109312) (width 0.25) (layer B.Cu) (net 6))
 (segment (start 146.812 101.693443) (end 146.31918 102.186263) (width 0.25) (layer B.Cu) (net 6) (status 20))
 (segment (start 146.812 100.33) (end 146.812 101.693443) (width 0.25) (layer B.Cu) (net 6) (status 10))
 (via (at 146.019181 102.486262) (size 0.6) (drill 0.4) (layers F.Cu B.Cu) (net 6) (status 30))
 (segment (start 146.31918 102.186263) (end 146.019181 102.486262) (width 0.25) (layer B.Cu) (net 6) (status 30))
 (segment (start 159.004 98.044) (end 157.15175 98.044) (width 0.25) (layer B.Cu) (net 10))
 (segment (start 157.15175 98.044) (end 156.889494 98.306256) (width 0.25) (layer B.Cu) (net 10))
 (segment (start 159.512 102.108) (end 159.512 98.552) (width 0.25) (layer F.Cu) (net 10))
 (segment (start 159.512 98.552) (end 159.004 98.044) (width 0.25) (layer F.Cu) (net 10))
 (via (at 159.004 98.044) (size 0.6) (drill 0.4) (layers F.Cu B.Cu) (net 10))
 (segment (start 159.004 102.616) (end 159.512 102.108) (width 0.25) (layer F.Cu) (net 10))
 (segment (start 160.02 103.298) (end 159.686 103.298) (width 0.25) (layer B.Cu) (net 10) (status 30))
 (segment (start 159.686 103.298) (end 159.004 102.616) (width 0.25) (layer B.Cu) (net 10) (status 10))
 (via (at 159.004 102.616) (size 0.6) (drill 0.4) (layers F.Cu B.Cu) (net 10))
 (segment (start 156.889494 97.709502) (end 156.889494 98.306256) (width 0.25) (layer F.Cu) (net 10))
 (segment (start 158.343599 93.573599) (end 158.343599 96.255397) (width 0.25) (layer F.Cu) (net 10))
 (segment (start 158.343599 96.255397) (end 156.889494 97.709502) (width 0.25) (layer F.Cu) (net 10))
 (segment (start 157.48 92.71) (end 158.343599 93.573599) (width 0.25) (layer F.Cu) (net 10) (status 10))
 (segment (start 156.186742 98.030975) (end 156.614213 98.030975) (width 0.25) (layer B.Cu) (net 10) (status 10))
 (via (at 156.889494 98.306256) (size 0.6) (drill 0.4) (layers F.Cu B.Cu) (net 10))
 (segment (start 156.614213 98.030975) (end 156.889494 98.306256) (width 0.25) (layer B.Cu) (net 10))
 (segment (start 159.846 108.204) (end 159.746 108.204) (width 0.25) (layer B.Cu) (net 8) (status 30))
 (segment (start 159.746 108.204) (end 159.238 107.696) (width 0.25) (layer B.Cu) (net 8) (status 30))
 (segment (start 161.036 94.488) (end 161.036 93.726) (width 0.25) (layer F.Cu) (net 8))
 (segment (start 161.036 93.726) (end 160.02 92.71) (width 0.25) (layer F.Cu) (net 8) (status 20))
 (segment (start 156.186742 97.041025) (end 158.482975 97.041025) (width 0.25) (layer B.Cu) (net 8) (status 10))
 (segment (start 158.482975 97.041025) (end 161.036 94.488) (width 0.25) (layer B.Cu) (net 8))
 (via (at 161.036 94.488) (size 0.6) (drill 0.4) (layers F.Cu B.Cu) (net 8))
 (segment (start 152.343876 95.602323) (end 152.343876 94.996) (width 0.25) (layer B.Cu) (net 13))
 (segment (start 152.343876 94.996) (end 152.343876 93.987438) (width 0.25) (layer B.Cu) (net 13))
 (segment (start 151.892 94.488) (end 152.343876 94.939876) (width 0.25) (layer B.Cu) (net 13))
 (segment (start 152.343876 94.939876) (end 152.343876 94.996) (width 0.25) (layer B.Cu) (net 13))
 (via (at 151.892 94.488) (size 0.6) (drill 0.4) (layers F.Cu B.Cu) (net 13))
 (segment (start 146.638 97.202) (end 149.352 94.488) (width 0.25) (layer F.Cu) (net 13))
 (segment (start 149.352 94.488) (end 151.892 94.488) (width 0.25) (layer F.Cu) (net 13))
 (segment (start 143.51 97.202) (end 146.638 97.202) (width 0.25) (layer F.Cu) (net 13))
 (segment (start 152.721918 95.980365) (end 152.343876 95.602323) (width 0.25) (layer B.Cu) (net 13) (status 10))
 (segment (start 152.343876 93.987438) (end 152.4 93.931314) (width 0.25) (layer B.Cu) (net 13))
 (segment (start 152.4 93.931314) (end 152.4 92.71) (width 0.25) (layer B.Cu) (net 13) (status 20))
 (via (at 143.51 97.202) (size 0.6) (drill 0.4) (layers F.Cu B.Cu) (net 13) (status 30))
 (segment (start 160.25513 91.186) (end 160.25513 90.40513) (width 0.25) (layer B.Cu) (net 7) (status 20))
 (segment (start 160.25513 90.40513) (end 160.02 90.17) (width 0.25) (layer B.Cu) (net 7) (status 30))
 (segment (start 161.29 93.19913) (end 161.29 92.22087) (width 0.25) (layer B.Cu) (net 7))
 (segment (start 161.29 92.22087) (end 160.25513 91.186) (width 0.25) (layer B.Cu) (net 7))
 (segment (start 155.833188 96.687472) (end 156.211231 96.309429) (width 0.25) (layer B.Cu) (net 7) (status 10))
 (segment (start 156.211231 96.309429) (end 158.179701 96.309429) (width 0.25) (layer B.Cu) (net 7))
 (segment (start 158.179701 96.309429) (end 161.29 93.19913) (width 0.25) (layer B.Cu) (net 7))
 (segment (start 158.668601 91.358601) (end 157.48 90.17) (width 0.25) (layer B.Cu) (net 9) (status 20))
 (segment (start 158.668601 93.280529) (end 158.668601 91.358601) (width 0.25) (layer B.Cu) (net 9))
 (segment (start 157.070132 94.878998) (end 158.668601 93.280529) (width 0.25) (layer B.Cu) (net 9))
 (segment (start 156.934555 94.878998) (end 157.070132 94.878998) (width 0.25) (layer B.Cu) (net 9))
 (segment (start 155.479635 96.333918) (end 156.934555 94.878998) (width 0.25) (layer B.Cu) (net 9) (status 10))
 (segment (start 155.126082 95.980365) (end 156.21 94.896447) (width 0.25) (layer B.Cu) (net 11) (status 10))
 (segment (start 156.21 94.896447) (end 156.21 91.44) (width 0.25) (layer B.Cu) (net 11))
 (segment (start 156.21 91.44) (end 154.94 90.17) (width 0.25) (layer B.Cu) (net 11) (status 20))
 (segment (start 154.772528 95.626812) (end 155.150571 95.248769) (width 0.25) (layer B.Cu) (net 12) (status 10))
 (segment (start 155.150571 95.248769) (end 155.150571 94.679701) (width 0.25) (layer B.Cu) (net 12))
 (segment (start 155.150571 94.679701) (end 153.588601 93.117731) (width 0.25) (layer B.Cu) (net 12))
 (segment (start 153.588601 93.117731) (end 153.588601 91.358601) (width 0.25) (layer B.Cu) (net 12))
 (segment (start 153.588601 91.358601) (end 152.4 90.17) (width 0.25) (layer B.Cu) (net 12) (status 20))
 (segment (start 151.211399 91.521399) (end 150.723599 91.033599) (width 0.25) (layer B.Cu) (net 14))
 (segment (start 151.298515 95.264068) (end 151.298515 94.819517) (width 0.25) (layer B.Cu) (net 14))
 (segment (start 151.298515 94.819517) (end 151.211399 94.732401) (width 0.25) (layer B.Cu) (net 14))
 (segment (start 152.368365 96.333918) (end 151.298515 95.264068) (width 0.25) (layer B.Cu) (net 14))
 (segment (start 150.723599 91.033599) (end 149.86 90.17) (width 0.25) (layer B.Cu) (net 14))
 (segment (start 151.211399 94.732401) (end 151.211399 91.521399) (width 0.25) (layer B.Cu) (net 14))
 (segment (start 148.183599 91.033599) (end 147.32 90.17) (width 0.25) (layer B.Cu) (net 15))
 (segment (start 148.671399 91.521399) (end 148.183599 91.033599) (width 0.25) (layer B.Cu) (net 15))
 (segment (start 151.065352 95.738012) (end 150.373512 95.738012) (width 0.25) (layer B.Cu) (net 15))
 (segment (start 152.014812 96.687472) (end 151.065352 95.738012) (width 0.25) (layer B.Cu) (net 15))
 (segment (start 148.671399 94.035899) (end 148.671399 91.521399) (width 0.25) (layer B.Cu) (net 15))
 (segment (start 150.373512 95.738012) (end 148.671399 94.035899) (width 0.25) (layer B.Cu) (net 15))
 (segment (start 145.643599 91.033599) (end 144.78 90.17) (width 0.25) (layer B.Cu) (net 16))
 (segment (start 149.038893 96.188023) (end 145.968601 93.117731) (width 0.25) (layer B.Cu) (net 16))
 (segment (start 150.808256 96.188023) (end 149.038893 96.188023) (width 0.25) (layer B.Cu) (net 16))
 (segment (start 145.968601 91.358601) (end 145.643599 91.033599) (width 0.25) (layer B.Cu) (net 16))
 (segment (start 151.661258 97.041025) (end 150.808256 96.188023) (width 0.25) (layer B.Cu) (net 16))
 (segment (start 145.968601 93.117731) (end 145.968601 91.358601) (width 0.25) (layer B.Cu) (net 16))
 (segment (start 143.591399 91.521399) (end 142.24 90.17) (width 0.25) (layer B.Cu) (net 17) (status 20))
 (segment (start 143.591399 93.280529) (end 143.591399 91.521399) (width 0.25) (layer B.Cu) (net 17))
 (segment (start 147.554889 97.244019) (end 143.591399 93.280529) (width 0.25) (layer B.Cu) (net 17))
 (segment (start 150.874302 97.244019) (end 147.554889 97.244019) (width 0.25) (layer B.Cu) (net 17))
 (segment (start 151.661258 98.030975) (end 150.874302 97.244019) (width 0.25) (layer B.Cu) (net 17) (status 10))
 (segment (start 159.004 94.488) (end 160.274 95.758) (width 0.25) (layer F.Cu) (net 2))
 (segment (start 160.274 95.758) (end 160.274 96.647) (width 0.25) (layer F.Cu) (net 2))
 (segment (start 157.353 95.631) (end 157.861 95.631) (width 0.25) (layer B.Cu) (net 2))
 (segment (start 157.861 95.631) (end 159.004 94.488) (width 0.25) (layer B.Cu) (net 2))
 (via (at 159.004 94.488) (size 0.6) (drill 0.4) (layers F.Cu B.Cu) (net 2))
 (segment (start 154.94 92.71) (end 157.353 95.123) (width 0.25) (layer F.Cu) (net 2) (status 10))
 (segment (start 157.353 95.123) (end 157.353 95.631) (width 0.25) (layer F.Cu) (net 2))
 (via (at 157.353 95.631) (size 0.6) (drill 0.4) (layers F.Cu B.Cu) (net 2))
 (segment (start 160.274 98.572) (end 160.274 96.647) (width 0.25) (layer B.Cu) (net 2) (status 10))
 (via (at 160.274 96.647) (size 0.6) (drill 0.4) (layers F.Cu B.Cu) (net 2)))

